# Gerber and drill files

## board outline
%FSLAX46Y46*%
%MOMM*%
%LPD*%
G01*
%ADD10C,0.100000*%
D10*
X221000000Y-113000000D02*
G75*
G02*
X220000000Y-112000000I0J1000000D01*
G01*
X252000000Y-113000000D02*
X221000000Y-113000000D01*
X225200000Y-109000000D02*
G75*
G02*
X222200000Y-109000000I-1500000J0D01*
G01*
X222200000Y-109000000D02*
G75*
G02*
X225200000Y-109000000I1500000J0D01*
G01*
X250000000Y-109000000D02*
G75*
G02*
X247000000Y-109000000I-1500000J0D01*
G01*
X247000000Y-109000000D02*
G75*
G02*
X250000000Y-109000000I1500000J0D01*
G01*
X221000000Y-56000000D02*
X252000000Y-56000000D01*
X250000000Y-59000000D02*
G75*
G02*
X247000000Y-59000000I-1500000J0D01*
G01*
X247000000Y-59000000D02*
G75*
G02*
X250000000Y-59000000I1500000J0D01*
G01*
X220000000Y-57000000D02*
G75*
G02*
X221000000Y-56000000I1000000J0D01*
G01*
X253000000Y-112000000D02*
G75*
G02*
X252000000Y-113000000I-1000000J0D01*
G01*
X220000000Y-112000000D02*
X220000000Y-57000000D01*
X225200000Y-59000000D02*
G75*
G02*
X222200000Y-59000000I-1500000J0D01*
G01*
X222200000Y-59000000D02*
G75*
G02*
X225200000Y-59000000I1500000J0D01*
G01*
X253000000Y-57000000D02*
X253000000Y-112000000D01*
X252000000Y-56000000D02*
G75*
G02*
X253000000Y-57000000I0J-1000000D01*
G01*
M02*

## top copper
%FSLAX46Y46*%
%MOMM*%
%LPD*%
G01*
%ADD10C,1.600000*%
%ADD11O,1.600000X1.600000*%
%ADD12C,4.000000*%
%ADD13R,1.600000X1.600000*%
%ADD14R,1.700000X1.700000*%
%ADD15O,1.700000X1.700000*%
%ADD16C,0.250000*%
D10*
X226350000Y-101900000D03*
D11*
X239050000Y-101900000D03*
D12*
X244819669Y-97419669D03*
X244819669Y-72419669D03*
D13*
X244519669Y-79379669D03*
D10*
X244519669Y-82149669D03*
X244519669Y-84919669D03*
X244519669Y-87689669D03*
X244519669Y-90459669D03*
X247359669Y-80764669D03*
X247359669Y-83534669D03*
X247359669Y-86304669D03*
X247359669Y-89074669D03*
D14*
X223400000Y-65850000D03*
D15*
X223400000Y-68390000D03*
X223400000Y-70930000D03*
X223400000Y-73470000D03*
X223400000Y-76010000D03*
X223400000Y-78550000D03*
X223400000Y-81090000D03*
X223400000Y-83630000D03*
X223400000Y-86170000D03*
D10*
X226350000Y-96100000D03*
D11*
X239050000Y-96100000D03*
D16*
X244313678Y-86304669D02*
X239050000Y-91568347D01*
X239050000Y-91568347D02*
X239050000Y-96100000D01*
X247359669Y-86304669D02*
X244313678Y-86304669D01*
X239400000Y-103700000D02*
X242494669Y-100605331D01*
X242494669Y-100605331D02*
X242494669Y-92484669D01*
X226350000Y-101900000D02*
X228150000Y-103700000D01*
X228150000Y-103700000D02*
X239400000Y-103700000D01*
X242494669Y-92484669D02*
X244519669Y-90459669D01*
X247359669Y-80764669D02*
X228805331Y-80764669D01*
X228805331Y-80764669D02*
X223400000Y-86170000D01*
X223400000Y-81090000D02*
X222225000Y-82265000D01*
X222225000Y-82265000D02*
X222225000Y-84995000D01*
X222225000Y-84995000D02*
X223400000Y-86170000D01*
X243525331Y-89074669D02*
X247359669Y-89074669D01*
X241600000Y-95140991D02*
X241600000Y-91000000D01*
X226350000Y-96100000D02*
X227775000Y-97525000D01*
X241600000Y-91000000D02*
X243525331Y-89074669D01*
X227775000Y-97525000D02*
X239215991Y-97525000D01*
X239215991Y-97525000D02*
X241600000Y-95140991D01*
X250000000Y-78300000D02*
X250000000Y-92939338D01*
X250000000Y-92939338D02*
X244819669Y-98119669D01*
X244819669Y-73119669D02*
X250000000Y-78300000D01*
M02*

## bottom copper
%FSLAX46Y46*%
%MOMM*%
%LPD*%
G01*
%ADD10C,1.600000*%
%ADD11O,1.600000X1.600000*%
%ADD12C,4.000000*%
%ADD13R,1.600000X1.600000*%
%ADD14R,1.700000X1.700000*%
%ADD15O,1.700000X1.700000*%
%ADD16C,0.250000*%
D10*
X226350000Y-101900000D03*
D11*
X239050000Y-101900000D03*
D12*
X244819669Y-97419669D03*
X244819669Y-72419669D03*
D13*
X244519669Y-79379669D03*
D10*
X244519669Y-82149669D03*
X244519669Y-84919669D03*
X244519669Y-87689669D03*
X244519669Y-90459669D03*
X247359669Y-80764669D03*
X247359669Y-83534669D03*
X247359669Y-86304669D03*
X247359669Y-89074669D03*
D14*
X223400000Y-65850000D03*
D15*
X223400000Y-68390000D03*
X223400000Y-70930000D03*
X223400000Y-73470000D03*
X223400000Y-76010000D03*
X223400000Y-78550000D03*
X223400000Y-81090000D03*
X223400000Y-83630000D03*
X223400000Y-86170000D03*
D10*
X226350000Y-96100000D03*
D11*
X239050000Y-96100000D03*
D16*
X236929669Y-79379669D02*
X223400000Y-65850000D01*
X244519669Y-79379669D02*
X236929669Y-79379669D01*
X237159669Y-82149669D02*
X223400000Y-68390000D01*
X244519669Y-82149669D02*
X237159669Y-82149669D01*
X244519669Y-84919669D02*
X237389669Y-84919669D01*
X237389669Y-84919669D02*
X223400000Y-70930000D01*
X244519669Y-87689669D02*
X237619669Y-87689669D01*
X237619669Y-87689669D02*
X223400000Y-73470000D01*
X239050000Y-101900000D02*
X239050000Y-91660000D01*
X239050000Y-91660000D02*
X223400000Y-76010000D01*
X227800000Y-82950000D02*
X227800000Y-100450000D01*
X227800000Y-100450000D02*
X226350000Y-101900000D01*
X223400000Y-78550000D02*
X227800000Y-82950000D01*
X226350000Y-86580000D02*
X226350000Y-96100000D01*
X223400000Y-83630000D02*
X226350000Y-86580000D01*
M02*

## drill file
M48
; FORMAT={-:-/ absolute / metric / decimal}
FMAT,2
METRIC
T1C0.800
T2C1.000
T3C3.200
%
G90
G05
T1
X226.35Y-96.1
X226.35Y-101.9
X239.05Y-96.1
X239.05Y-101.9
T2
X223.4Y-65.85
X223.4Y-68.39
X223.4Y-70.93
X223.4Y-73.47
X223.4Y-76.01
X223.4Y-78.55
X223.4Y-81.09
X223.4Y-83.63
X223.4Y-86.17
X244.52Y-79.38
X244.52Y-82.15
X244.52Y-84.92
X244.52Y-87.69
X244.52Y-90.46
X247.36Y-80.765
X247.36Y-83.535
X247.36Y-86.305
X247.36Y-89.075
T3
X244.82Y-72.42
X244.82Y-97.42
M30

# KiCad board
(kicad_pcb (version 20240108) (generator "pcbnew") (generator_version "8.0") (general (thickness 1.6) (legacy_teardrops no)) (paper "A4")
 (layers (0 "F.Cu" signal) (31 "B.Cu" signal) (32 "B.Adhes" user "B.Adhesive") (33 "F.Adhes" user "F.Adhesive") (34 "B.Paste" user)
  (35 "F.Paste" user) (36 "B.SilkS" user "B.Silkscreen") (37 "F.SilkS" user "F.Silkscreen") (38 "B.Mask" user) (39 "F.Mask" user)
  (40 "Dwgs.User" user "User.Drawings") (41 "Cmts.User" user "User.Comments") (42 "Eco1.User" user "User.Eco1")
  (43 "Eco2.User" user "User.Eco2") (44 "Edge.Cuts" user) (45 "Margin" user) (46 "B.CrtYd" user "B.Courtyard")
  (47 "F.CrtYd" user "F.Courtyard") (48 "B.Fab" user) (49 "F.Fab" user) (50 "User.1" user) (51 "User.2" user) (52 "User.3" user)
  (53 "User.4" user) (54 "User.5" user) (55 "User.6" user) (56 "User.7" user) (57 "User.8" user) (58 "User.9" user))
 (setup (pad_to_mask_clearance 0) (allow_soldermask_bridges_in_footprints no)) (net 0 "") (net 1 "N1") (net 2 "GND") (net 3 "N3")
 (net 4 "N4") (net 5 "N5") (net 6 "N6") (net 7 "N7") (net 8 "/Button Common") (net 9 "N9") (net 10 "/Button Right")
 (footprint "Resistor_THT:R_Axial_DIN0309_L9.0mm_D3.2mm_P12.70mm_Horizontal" (layer "F.Cu") (at 226.35 101.9)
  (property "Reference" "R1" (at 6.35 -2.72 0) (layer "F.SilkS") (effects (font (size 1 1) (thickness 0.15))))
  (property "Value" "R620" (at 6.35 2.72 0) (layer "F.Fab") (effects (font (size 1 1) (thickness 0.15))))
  (pad "1" thru_hole circle (at 0 0) (size 1.6 1.6) (drill 0.8) (layers "*.Cu" "*.Mask") (remove_unused_layers no) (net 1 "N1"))
  (pad "2" thru_hole oval (at 12.7 0) (size 1.6 1.6) (drill 0.8) (layers "*.Cu" "*.Mask") (remove_unused_layers no) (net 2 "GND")))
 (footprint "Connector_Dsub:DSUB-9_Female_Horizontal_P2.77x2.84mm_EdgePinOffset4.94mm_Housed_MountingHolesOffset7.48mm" (layer "F.Cu")
  (at 244.519669 79.379669 90)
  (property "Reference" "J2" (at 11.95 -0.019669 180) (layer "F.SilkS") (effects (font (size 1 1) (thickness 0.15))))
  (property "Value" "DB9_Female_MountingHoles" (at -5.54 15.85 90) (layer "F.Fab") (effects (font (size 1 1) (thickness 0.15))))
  (pad "0" thru_hole circle (at -18.04 0.3 90) (size 4 4) (drill 3.2) (layers "*.Cu" "*.Mask") (remove_unused_layers no) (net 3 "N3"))
  (pad "0" thru_hole circle (at 6.96 0.3 90) (size 4 4) (drill 3.2) (layers "*.Cu" "*.Mask") (remove_unused_layers no) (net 3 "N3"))
  (pad "1" thru_hole rect (at 0 0 90) (size 1.6 1.6) (drill 1) (layers "*.Cu" "*.Mask") (remove_unused_layers no) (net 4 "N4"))
  (pad "2" thru_hole circle (at -2.77 0 90) (size 1.6 1.6) (drill 1) (layers "*.Cu" "*.Mask") (remove_unused_layers no) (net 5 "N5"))
  (pad "3" thru_hole circle (at -5.54 0 90) (size 1.6 1.6) (drill 1) (layers "*.Cu" "*.Mask") (remove_unused_layers no) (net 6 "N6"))
  (pad "4" thru_hole circle (at -8.31 0 90) (size 1.6 1.6) (drill 1) (layers "*.Cu" "*.Mask") (remove_unused_layers no) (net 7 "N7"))
  (pad "5" thru_hole circle (at -11.08 0 90) (size 1.6 1.6) (drill 1) (layers "*.Cu" "*.Mask") (remove_unused_layers no) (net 1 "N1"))
  (pad "6" thru_hole circle (at -1.385 2.84 90) (size 1.6 1.6) (drill 1) (layers "*.Cu" "*.Mask") (remove_unused_layers no)
   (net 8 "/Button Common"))
  (pad "7" thru_hole circle (at -4.155 2.84 90) (size 1.6 1.6) (drill 1) (layers "*.Cu" "*.Mask") (remove_unused_layers no) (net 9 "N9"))
  (pad "8" thru_hole circle (at -6.925 2.84 90) (size 1.6 1.6) (drill 1) (layers "*.Cu" "*.Mask") (remove_unused_layers no) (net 2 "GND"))
  (pad "9" thru_hole circle (at -9.695 2.84 90) (size 1.6 1.6) (drill 1) (layers "*.Cu" "*.Mask") (remove_unused_layers no)
   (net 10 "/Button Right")))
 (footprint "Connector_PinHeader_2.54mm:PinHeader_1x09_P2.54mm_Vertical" (layer "F.Cu") (at 223.4 65.85)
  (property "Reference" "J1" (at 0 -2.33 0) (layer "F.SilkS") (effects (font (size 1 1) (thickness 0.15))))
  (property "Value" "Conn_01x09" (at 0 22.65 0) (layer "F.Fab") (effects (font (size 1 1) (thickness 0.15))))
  (pad "1" thru_hole rect (at 0 0) (size 1.7 1.7) (drill 1) (layers "*.Cu" "*.Mask") (remove_unused_layers no) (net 4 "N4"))
  (pad "2" thru_hole oval (at 0 2.54) (size 1.7 1.7) (drill 1) (layers "*.Cu" "*.Mask") (remove_unused_layers no) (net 5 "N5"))
  (pad "3" thru_hole oval (at 0 5.08) (size 1.7 1.7) (drill 1) (layers "*.Cu" "*.Mask") (remove_unused_layers no) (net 6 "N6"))
  (pad "4" thru_hole oval (at 0 7.62) (size 1.7 1.7) (drill 1) (layers "*.Cu" "*.Mask") (remove_unused_layers no) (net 7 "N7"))
  (pad "5" thru_hole oval (at 0 10.16) (size 1.7 1.7) (drill 1) (layers "*.Cu" "*.Mask") (remove_unused_layers no) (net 2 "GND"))
  (pad "6" thru_hole oval (at 0 12.7) (size 1.7 1.7) (drill 1) (layers "*.Cu" "*.Mask") (remove_unused_layers no) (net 1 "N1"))
  (pad "7" thru_hole oval (at 0 15.24) (size 1.7 1.7) (drill 1) (layers "*.Cu" "*.Mask") (remove_unused_layers no) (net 8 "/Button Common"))
  (pad "8" thru_hole oval (at 0 17.78) (size 1.7 1.7) (drill 1) (layers "*.Cu" "*.Mask") (remove_unused_layers no) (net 10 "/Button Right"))
  (pad "9" thru_hole oval (at 0 20.32) (size 1.7 1.7) (drill 1) (layers "*.Cu" "*.Mask") (remove_unused_layers no) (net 8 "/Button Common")))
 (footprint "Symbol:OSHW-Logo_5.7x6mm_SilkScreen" (layer "F.Cu") (at 234.9 59.9)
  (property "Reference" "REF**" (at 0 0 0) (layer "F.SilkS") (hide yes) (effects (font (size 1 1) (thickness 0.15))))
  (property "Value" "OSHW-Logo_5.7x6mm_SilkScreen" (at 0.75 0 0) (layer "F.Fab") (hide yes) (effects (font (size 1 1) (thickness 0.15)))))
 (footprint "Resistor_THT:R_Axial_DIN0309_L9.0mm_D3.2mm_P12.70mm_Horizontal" (layer "F.Cu") (at 226.35 96.1)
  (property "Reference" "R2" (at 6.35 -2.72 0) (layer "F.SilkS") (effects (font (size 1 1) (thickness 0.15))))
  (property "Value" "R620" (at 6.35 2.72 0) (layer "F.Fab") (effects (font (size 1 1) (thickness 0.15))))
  (pad "1" thru_hole circle (at 0 0) (size 1.6 1.6) (drill 0.8) (layers "*.Cu" "*.Mask") (remove_unused_layers no) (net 10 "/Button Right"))
  (pad "2" thru_hole oval (at 12.7 0) (size 1.6 1.6) (drill 0.8) (layers "*.Cu" "*.Mask") (remove_unused_layers no) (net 2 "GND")))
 (gr_arc (start 221 113) (mid 220.292893 112.707107) (end 220 112) (stroke (width 0.1) (type solid)) (layer "Edge.Cuts"))
 (gr_line (start 252 113) (end 221 113) (stroke (width 0.1) (type solid)) (layer "Edge.Cuts"))
 (gr_circle (center 223.7 109) (end 225.2 109) (stroke (width 0.1) (type solid)) (fill none) (layer "Edge.Cuts"))
 (gr_circle (center 248.5 109) (end 250 109) (stroke (width 0.1) (type solid)) (fill none) (layer "Edge.Cuts"))
 (gr_line (start 221 56) (end 252 56) (stroke (width 0.1) (type solid)) (layer "Edge.Cuts"))
 (gr_circle (center 248.5 59) (end 250 59) (stroke (width 0.1) (type solid)) (fill none) (layer "Edge.Cuts"))
 (gr_arc (start 220 57) (mid 220.292893 56.292893) (end 221 56) (stroke (width 0.1) (type solid)) (layer "Edge.Cuts"))
 (gr_arc (start 253 112) (mid 252.707107 112.707107) (end 252 113) (stroke (width 0.1) (type solid)) (layer "Edge.Cuts"))
 (gr_line (start 220 112) (end 220 57) (stroke (width 0.1) (type solid)) (layer "Edge.Cuts"))
 (gr_circle (center 223.7 59) (end 225.2 59) (stroke (width 0.1) (type solid)) (fill none) (layer "Edge.Cuts"))
 (gr_line (start 253 57) (end 253 112) (stroke (width 0.1) (type solid)) (layer "Edge.Cuts"))
 (gr_arc (start 252 56) (mid 252.707107 56.292893) (end 253 57) (stroke (width 0.1) (type solid)) (layer "Edge.Cuts"))
 (segment (start 236.929669 79.379669) (end 223.4 65.85) (width 0.25) (layer "B.Cu") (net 4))
 (segment (start 244.519669 79.379669) (end 236.929669 79.379669) (width 0.25) (layer "B.Cu") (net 4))
 (segment (start 237.159669 82.149669) (end 223.4 68.39) (width 0.25) (layer "B.Cu") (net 5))
 (segment (start 244.519669 82.149669) (end 237.159669 82.149669) (width 0.25) (layer "B.Cu") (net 5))
 (segment (start 244.519669 84.919669) (end 237.389669 84.919669) (width 0.25) (layer "B.Cu") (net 6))
 (segment (start 237.389669 84.919669) (end 223.4 70.93) (width 0.25) (layer "B.Cu") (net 6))
 (segment (start 244.519669 87.689669) (end 237.619669 87.689669) (width 0.25) (layer "B.Cu") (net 7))
 (segment (start 237.619669 87.689669) (end 223.4 73.47) (width 0.25) (layer "B.Cu") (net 7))
 (segment (start 244.313678 86.304669) (end 239.05 91.568347) (width 0.25) (layer "F.Cu") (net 2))
 (segment (start 239.05 91.568347) (end 239.05 96.1) (width 0.25) (layer "F.Cu") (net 2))
 (segment (start 247.359669 86.304669) (end 244.313678 86.304669) (width 0.25) (layer "F.Cu") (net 2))
 (segment (start 239.05 101.9) (end 239.05 91.66) (width 0.25) (layer "B.Cu") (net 2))
 (segment (start 239.05 91.66) (end 223.4 76.01) (width 0.25) (layer "B.Cu") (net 2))
 (segment (start 239.4 103.7) (end 242.494669 100.605331) (width 0.25) (layer "F.Cu") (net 1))
 (segment (start 242.494669 100.605331) (end 242.494669 92.484669) (width 0.25) (layer "F.Cu") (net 1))
 (segment (start 226.35 101.9) (end 228.15 103.7) (width 0.25) (layer "F.Cu") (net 1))
 (segment (start 228.15 103.7) (end 239.4 103.7) (width 0.25) (layer "F.Cu") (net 1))
 (segment (start 242.494669 92.484669) (end 244.519669 90.459669) (width 0.25) (layer "F.Cu") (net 1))
 (segment (start 227.8 82.95) (end 227.8 100.45) (width 0.25) (layer "B.Cu") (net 1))
 (segment (start 227.8 100.45) (end 226.35 101.9) (width 0.25) (layer "B.Cu") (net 1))
 (segment (start 223.4 78.55) (end 227.8 82.95) (width 0.25) (layer "B.Cu") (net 1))
 (segment (start 247.359669 80.764669) (end 228.805331 80.764669) (width 0.25) (layer "F.Cu") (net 8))
 (segment (start 228.805331 80.764669) (end 223.4 86.17) (width 0.25) (layer "F.Cu") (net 8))
 (segment (start 223.4 81.09) (end 222.225 82.265) (width 0.25) (layer "F.Cu") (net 8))
 (segment (start 222.225 82.265) (end 222.225 84.995) (width 0.25) (layer "F.Cu") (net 8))
 (segment (start 222.225 84.995) (end 223.4 86.17) (width 0.25) (layer "F.Cu") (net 8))
 (segment (start 243.525331 89.074669) (end 247.359669 89.074669) (width 0.25) (layer "F.Cu") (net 10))
 (segment (start 241.6 95.140991) (end 241.6 91) (width 0.25) (layer "F.Cu") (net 10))
 (segment (start 226.35 96.1) (end 227.775 97.525) (width 0.25) (layer "F.Cu") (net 10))
 (segment (start 241.6 91) (end 243.525331 89.074669) (width 0.25) (layer "F.Cu") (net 10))
 (segment (start 227.775 97.525) (end 239.215991 97.525) (width 0.25) (layer "F.Cu") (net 10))
 (segment (start 239.215991 97.525) (end 241.6 95.140991) (width 0.25) (layer "F.Cu") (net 10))
 (segment (start 226.35 86.58) (end 226.35 96.1) (width 0.25) (layer "B.Cu") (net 10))
 (segment (start 223.4 83.63) (end 226.35 86.58) (width 0.25) (layer "B.Cu") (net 10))
 (segment (start 250 78.3) (end 250 92.939338) (width 0.25) (layer "F.Cu") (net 3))
 (segment (start 250 92.939338) (end 244.819669 98.119669) (width 0.25) (layer "F.Cu") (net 3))
 (segment (start 244.819669 73.119669) (end 250 78.3) (width 0.25) (layer "F.Cu") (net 3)))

